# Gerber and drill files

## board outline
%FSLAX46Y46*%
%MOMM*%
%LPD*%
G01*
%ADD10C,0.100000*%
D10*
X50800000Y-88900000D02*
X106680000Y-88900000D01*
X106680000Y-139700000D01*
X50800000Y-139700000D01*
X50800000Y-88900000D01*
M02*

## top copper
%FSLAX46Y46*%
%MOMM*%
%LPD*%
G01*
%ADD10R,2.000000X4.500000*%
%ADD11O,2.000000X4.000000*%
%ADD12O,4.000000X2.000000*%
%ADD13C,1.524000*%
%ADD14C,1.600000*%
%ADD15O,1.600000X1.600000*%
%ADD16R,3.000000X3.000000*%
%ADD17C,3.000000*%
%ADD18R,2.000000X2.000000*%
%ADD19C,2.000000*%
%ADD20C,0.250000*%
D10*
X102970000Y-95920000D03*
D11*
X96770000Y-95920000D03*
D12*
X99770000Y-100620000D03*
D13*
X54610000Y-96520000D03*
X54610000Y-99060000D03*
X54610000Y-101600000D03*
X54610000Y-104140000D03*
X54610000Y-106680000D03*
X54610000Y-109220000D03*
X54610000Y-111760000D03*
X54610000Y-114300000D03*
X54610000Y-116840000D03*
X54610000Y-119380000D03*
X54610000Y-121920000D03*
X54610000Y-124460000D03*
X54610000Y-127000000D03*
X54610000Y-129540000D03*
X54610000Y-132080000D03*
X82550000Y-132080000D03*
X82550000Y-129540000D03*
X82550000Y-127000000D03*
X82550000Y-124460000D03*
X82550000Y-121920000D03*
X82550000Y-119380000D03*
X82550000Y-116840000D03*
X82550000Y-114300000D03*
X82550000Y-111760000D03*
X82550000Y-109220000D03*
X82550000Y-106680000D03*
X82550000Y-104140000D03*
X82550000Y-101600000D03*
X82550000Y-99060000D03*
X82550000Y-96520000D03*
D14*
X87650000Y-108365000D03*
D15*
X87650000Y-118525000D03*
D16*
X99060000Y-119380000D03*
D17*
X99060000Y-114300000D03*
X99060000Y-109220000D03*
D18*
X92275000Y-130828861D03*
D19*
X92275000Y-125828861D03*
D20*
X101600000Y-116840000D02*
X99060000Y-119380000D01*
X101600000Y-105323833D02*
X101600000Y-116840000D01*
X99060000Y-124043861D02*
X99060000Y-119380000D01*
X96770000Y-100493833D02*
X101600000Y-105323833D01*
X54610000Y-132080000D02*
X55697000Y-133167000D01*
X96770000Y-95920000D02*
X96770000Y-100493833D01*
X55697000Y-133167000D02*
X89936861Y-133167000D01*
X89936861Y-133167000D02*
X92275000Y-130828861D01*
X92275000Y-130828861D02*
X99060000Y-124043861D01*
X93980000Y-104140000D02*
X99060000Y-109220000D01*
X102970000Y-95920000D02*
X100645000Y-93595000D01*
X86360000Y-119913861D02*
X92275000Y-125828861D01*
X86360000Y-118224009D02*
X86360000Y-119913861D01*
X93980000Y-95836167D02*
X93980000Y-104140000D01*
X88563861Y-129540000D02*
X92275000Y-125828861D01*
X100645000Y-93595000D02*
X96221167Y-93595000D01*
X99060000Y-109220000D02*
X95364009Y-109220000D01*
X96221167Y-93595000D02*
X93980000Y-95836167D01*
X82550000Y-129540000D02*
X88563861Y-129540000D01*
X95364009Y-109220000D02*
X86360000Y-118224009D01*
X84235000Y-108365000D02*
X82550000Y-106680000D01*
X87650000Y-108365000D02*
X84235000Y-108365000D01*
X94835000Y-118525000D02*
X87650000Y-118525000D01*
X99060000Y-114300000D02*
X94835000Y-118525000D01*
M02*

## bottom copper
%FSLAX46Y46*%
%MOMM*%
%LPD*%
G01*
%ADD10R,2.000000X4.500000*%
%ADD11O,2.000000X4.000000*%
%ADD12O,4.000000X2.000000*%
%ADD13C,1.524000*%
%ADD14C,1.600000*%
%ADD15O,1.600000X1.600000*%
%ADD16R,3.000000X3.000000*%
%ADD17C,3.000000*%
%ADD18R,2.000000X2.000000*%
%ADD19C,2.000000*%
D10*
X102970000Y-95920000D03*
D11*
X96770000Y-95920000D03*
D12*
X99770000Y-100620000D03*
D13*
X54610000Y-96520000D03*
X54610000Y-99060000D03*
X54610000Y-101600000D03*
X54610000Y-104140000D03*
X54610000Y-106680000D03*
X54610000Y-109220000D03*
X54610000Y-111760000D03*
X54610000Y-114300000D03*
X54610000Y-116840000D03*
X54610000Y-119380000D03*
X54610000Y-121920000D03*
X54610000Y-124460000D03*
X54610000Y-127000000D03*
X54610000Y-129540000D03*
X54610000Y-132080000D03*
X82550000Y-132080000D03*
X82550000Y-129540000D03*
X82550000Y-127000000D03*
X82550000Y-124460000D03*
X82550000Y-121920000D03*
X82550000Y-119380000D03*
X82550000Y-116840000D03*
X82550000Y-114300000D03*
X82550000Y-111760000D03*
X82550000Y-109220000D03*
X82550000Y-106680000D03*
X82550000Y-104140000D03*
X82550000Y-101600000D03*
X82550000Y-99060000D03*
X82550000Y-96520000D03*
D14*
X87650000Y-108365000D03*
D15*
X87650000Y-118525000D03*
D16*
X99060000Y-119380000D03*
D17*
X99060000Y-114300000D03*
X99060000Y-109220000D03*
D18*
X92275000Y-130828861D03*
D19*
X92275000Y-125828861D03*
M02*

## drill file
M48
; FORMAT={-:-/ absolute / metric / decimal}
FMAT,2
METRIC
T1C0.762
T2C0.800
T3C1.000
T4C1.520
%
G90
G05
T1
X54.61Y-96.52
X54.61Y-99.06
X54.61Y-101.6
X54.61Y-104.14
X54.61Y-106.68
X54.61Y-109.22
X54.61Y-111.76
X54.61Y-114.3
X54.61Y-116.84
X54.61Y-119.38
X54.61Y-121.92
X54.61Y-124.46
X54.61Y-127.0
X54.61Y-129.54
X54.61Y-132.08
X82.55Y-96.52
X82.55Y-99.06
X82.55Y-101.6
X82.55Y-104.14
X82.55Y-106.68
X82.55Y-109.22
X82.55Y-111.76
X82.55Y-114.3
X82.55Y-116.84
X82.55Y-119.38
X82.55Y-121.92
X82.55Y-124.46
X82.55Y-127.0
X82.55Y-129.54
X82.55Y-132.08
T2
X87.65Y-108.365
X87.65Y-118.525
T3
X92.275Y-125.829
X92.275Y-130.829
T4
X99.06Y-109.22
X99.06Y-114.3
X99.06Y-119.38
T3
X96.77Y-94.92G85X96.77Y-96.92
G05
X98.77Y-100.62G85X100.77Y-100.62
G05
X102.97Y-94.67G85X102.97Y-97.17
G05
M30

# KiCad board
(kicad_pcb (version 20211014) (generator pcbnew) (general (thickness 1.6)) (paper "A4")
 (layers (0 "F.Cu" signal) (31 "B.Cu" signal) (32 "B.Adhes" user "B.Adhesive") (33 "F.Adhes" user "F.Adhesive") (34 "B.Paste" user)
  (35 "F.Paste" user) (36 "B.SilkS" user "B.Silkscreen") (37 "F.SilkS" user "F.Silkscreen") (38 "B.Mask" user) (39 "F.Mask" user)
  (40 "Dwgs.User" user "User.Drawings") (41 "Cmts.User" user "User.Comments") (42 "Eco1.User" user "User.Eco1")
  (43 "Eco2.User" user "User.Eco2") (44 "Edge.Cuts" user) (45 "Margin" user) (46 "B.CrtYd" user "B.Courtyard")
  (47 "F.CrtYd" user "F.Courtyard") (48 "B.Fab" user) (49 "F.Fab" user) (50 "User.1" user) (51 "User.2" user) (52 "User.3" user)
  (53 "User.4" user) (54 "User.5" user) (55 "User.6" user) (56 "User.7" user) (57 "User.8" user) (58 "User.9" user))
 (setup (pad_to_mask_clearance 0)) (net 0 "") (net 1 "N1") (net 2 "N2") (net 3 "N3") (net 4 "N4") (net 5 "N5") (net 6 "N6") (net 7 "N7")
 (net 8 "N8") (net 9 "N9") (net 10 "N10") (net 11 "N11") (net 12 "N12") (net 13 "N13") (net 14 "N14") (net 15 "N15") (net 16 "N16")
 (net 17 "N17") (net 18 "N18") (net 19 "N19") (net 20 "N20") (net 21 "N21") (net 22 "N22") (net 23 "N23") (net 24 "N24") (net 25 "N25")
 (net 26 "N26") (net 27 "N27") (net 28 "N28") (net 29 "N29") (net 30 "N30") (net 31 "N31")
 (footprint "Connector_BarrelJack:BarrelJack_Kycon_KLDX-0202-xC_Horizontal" (layer "F.Cu") (at 102.97 95.92)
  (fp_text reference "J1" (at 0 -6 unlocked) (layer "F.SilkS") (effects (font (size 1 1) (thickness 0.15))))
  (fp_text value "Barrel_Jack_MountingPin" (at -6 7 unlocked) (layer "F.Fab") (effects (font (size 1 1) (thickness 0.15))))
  (pad "1" thru_hole rect (at 0 0) (size 2 4.5) (drill oval 1 3.5) (layers *.Cu *.Mask) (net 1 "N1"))
  (pad "2" thru_hole oval (at -6.2 0) (size 2 4) (drill oval 1 3) (layers *.Cu *.Mask) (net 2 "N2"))
  (pad "3" thru_hole oval (at -3.2 4.7 90) (size 2 4) (drill oval 1 3) (layers *.Cu *.Mask)))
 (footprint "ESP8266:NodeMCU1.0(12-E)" (layer "F.Cu") (at 68.58 114.3)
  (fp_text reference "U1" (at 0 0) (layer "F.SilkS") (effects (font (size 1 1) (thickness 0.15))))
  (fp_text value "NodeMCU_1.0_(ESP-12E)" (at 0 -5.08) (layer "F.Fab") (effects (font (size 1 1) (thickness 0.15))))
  (pad "1" thru_hole circle locked (at -13.97 -17.78) (size 1.524 1.524) (drill 0.762) (layers *.Cu *.Mask "F.SilkS") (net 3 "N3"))
  (pad "2" thru_hole circle locked (at -13.97 -15.24) (size 1.524 1.524) (drill 0.762) (layers *.Cu *.Mask "F.SilkS") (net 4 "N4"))
  (pad "3" thru_hole circle locked (at -13.97 -12.7) (size 1.524 1.524) (drill 0.762) (layers *.Cu *.Mask "F.SilkS") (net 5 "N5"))
  (pad "4" thru_hole circle locked (at -13.97 -10.16) (size 1.524 1.524) (drill 0.762) (layers *.Cu *.Mask "F.SilkS") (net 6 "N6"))
  (pad "5" thru_hole circle locked (at -13.97 -7.62) (size 1.524 1.524) (drill 0.762) (layers *.Cu *.Mask "F.SilkS") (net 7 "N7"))
  (pad "6" thru_hole circle locked (at -13.97 -5.08) (size 1.524 1.524) (drill 0.762) (layers *.Cu *.Mask "F.SilkS") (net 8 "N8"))
  (pad "7" thru_hole circle locked (at -13.97 -2.54) (size 1.524 1.524) (drill 0.762) (layers *.Cu *.Mask "F.SilkS") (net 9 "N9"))
  (pad "8" thru_hole circle locked (at -13.97 0) (size 1.524 1.524) (drill 0.762) (layers *.Cu *.Mask "F.SilkS") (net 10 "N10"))
  (pad "9" thru_hole circle locked (at -13.97 2.54) (size 1.524 1.524) (drill 0.762) (layers *.Cu *.Mask "F.SilkS") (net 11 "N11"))
  (pad "10" thru_hole circle locked (at -13.97 5.08) (size 1.524 1.524) (drill 0.762) (layers *.Cu *.Mask "F.SilkS") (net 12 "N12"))
  (pad "11" thru_hole circle locked (at -13.97 7.62) (size 1.524 1.524) (drill 0.762) (layers *.Cu *.Mask "F.SilkS") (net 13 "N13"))
  (pad "12" thru_hole circle locked (at -13.97 10.16) (size 1.524 1.524) (drill 0.762) (layers *.Cu *.Mask "F.SilkS") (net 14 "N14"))
  (pad "13" thru_hole circle locked (at -13.97 12.7) (size 1.524 1.524) (drill 0.762) (layers *.Cu *.Mask "F.SilkS") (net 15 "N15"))
  (pad "14" thru_hole circle locked (at -13.97 15.24) (size 1.524 1.524) (drill 0.762) (layers *.Cu *.Mask "F.SilkS") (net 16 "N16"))
  (pad "15" thru_hole circle locked (at -13.97 17.78) (size 1.524 1.524) (drill 0.762) (layers *.Cu *.Mask "F.SilkS") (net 2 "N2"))
  (pad "16" thru_hole circle locked (at 13.97 17.78) (size 1.524 1.524) (drill 0.762) (layers *.Cu *.Mask "F.SilkS") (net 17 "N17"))
  (pad "17" thru_hole circle locked (at 13.97 15.24) (size 1.524 1.524) (drill 0.762) (layers *.Cu *.Mask "F.SilkS") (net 1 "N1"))
  (pad "18" thru_hole circle locked (at 13.97 12.7) (size 1.524 1.524) (drill 0.762) (layers *.Cu *.Mask "F.SilkS") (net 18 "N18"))
  (pad "19" thru_hole circle locked (at 13.97 10.16) (size 1.524 1.524) (drill 0.762) (layers *.Cu *.Mask "F.SilkS") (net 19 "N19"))
  (pad "20" thru_hole circle locked (at 13.97 7.62) (size 1.524 1.524) (drill 0.762) (layers *.Cu *.Mask "F.SilkS") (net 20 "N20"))
  (pad "21" thru_hole circle locked (at 13.97 5.08) (size 1.524 1.524) (drill 0.762) (layers *.Cu *.Mask "F.SilkS") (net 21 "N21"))
  (pad "22" thru_hole circle locked (at 13.97 2.54) (size 1.524 1.524) (drill 0.762) (layers *.Cu *.Mask "F.SilkS") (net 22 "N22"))
  (pad "23" thru_hole circle locked (at 13.97 0) (size 1.524 1.524) (drill 0.762) (layers *.Cu *.Mask "F.SilkS") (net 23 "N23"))
  (pad "24" thru_hole circle locked (at 13.97 -2.54) (size 1.524 1.524) (drill 0.762) (layers *.Cu *.Mask "F.SilkS") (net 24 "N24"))
  (pad "25" thru_hole circle locked (at 13.97 -5.08) (size 1.524 1.524) (drill 0.762) (layers *.Cu *.Mask "F.SilkS") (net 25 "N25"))
  (pad "26" thru_hole circle locked (at 13.97 -7.62) (size 1.524 1.524) (drill 0.762) (layers *.Cu *.Mask "F.SilkS") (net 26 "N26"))
  (pad "27" thru_hole circle locked (at 13.97 -10.16) (size 1.524 1.524) (drill 0.762) (layers *.Cu *.Mask "F.SilkS") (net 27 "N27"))
  (pad "28" thru_hole circle locked (at 13.97 -12.7) (size 1.524 1.524) (drill 0.762) (layers *.Cu *.Mask "F.SilkS") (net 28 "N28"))
  (pad "29" thru_hole circle locked (at 13.97 -15.24) (size 1.524 1.524) (drill 0.762) (layers *.Cu *.Mask "F.SilkS") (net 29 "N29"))
  (pad "30" thru_hole circle locked (at 13.97 -17.78) (size 1.524 1.524) (drill 0.762) (layers *.Cu *.Mask "F.SilkS") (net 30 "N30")))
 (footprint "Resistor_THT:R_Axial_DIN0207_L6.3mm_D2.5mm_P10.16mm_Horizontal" (layer "F.Cu") (at 87.65 108.365 -90)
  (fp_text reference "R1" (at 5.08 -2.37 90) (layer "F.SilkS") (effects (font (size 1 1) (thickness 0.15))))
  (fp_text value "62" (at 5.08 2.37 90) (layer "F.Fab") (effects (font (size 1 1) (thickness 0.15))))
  (pad "1" thru_hole circle (at 0 0 270) (size 1.6 1.6) (drill 0.8) (layers *.Cu *.Mask) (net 26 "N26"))
  (pad "2" thru_hole oval (at 10.16 0 270) (size 1.6 1.6) (drill 0.8) (layers *.Cu *.Mask) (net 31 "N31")))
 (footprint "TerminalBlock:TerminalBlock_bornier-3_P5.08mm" (layer "F.Cu") (at 99.06 119.38 90)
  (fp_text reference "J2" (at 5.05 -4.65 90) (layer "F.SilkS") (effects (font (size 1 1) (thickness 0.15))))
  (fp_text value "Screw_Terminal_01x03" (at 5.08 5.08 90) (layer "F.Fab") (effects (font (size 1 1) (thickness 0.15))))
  (pad "1" thru_hole rect (at 0 0 90) (size 3 3) (drill 1.52) (layers *.Cu *.Mask) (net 2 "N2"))
  (pad "2" thru_hole circle (at 5.08 0 90) (size 3 3) (drill 1.52) (layers *.Cu *.Mask) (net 31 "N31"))
  (pad "3" thru_hole circle (at 10.16 0 90) (size 3 3) (drill 1.52) (layers *.Cu *.Mask) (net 1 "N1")))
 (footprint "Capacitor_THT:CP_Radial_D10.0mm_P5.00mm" (layer "F.Cu") (at 92.275 130.828861 90)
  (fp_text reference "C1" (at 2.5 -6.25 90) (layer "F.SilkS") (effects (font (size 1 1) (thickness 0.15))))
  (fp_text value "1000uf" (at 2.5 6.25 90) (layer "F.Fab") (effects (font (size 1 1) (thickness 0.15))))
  (pad "1" thru_hole rect (at 0 0 90) (size 2 2) (drill 1) (layers *.Cu *.Mask) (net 2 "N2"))
  (pad "2" thru_hole circle (at 5 0 90) (size 2 2) (drill 1) (layers *.Cu *.Mask) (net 1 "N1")))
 (gr_rect (start 50.8 88.9) (end 106.68 139.7) (layer "Edge.Cuts") (width 0.1) (fill none))
 (segment (start 101.6 116.84) (end 99.06 119.38) (width 0.25) (layer "F.Cu") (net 2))
 (segment (start 101.6 105.323833) (end 101.6 116.84) (width 0.25) (layer "F.Cu") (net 2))
 (segment (start 99.06 124.043861) (end 99.06 119.38) (width 0.25) (layer "F.Cu") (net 2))
 (segment (start 96.77 100.493833) (end 101.6 105.323833) (width 0.25) (layer "F.Cu") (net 2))
 (segment (start 54.61 132.08) (end 55.697 133.167) (width 0.25) (layer "F.Cu") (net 2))
 (segment (start 96.77 95.92) (end 96.77 100.493833) (width 0.25) (layer "F.Cu") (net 2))
 (segment (start 55.697 133.167) (end 89.936861 133.167) (width 0.25) (layer "F.Cu") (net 2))
 (segment (start 89.936861 133.167) (end 92.275 130.828861) (width 0.25) (layer "F.Cu") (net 2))
 (segment (start 92.275 130.828861) (end 99.06 124.043861) (width 0.25) (layer "F.Cu") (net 2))
 (segment (start 93.98 104.14) (end 99.06 109.22) (width 0.25) (layer "F.Cu") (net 1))
 (segment (start 102.97 95.92) (end 100.645 93.595) (width 0.25) (layer "F.Cu") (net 1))
 (segment (start 86.36 119.913861) (end 92.275 125.828861) (width 0.25) (layer "F.Cu") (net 1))
 (segment (start 86.36 118.224009) (end 86.36 119.913861) (width 0.25) (layer "F.Cu") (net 1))
 (segment (start 93.98 95.836167) (end 93.98 104.14) (width 0.25) (layer "F.Cu") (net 1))
 (segment (start 88.563861 129.54) (end 92.275 125.828861) (width 0.25) (layer "F.Cu") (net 1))
 (segment (start 100.645 93.595) (end 96.221167 93.595) (width 0.25) (layer "F.Cu") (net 1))
 (segment (start 99.06 109.22) (end 95.364009 109.22) (width 0.25) (layer "F.Cu") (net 1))
 (segment (start 96.221167 93.595) (end 93.98 95.836167) (width 0.25) (layer "F.Cu") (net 1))
 (segment (start 82.55 129.54) (end 88.563861 129.54) (width 0.25) (layer "F.Cu") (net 1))
 (segment (start 95.364009 109.22) (end 86.36 118.224009) (width 0.25) (layer "F.Cu") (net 1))
 (segment (start 84.235 108.365) (end 82.55 106.68) (width 0.25) (layer "F.Cu") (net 26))
 (segment (start 87.65 108.365) (end 84.235 108.365) (width 0.25) (layer "F.Cu") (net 26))
 (segment (start 94.835 118.525) (end 87.65 118.525) (width 0.25) (layer "F.Cu") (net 31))
 (segment (start 99.06 114.3) (end 94.835 118.525) (width 0.25) (layer "F.Cu") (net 31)))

